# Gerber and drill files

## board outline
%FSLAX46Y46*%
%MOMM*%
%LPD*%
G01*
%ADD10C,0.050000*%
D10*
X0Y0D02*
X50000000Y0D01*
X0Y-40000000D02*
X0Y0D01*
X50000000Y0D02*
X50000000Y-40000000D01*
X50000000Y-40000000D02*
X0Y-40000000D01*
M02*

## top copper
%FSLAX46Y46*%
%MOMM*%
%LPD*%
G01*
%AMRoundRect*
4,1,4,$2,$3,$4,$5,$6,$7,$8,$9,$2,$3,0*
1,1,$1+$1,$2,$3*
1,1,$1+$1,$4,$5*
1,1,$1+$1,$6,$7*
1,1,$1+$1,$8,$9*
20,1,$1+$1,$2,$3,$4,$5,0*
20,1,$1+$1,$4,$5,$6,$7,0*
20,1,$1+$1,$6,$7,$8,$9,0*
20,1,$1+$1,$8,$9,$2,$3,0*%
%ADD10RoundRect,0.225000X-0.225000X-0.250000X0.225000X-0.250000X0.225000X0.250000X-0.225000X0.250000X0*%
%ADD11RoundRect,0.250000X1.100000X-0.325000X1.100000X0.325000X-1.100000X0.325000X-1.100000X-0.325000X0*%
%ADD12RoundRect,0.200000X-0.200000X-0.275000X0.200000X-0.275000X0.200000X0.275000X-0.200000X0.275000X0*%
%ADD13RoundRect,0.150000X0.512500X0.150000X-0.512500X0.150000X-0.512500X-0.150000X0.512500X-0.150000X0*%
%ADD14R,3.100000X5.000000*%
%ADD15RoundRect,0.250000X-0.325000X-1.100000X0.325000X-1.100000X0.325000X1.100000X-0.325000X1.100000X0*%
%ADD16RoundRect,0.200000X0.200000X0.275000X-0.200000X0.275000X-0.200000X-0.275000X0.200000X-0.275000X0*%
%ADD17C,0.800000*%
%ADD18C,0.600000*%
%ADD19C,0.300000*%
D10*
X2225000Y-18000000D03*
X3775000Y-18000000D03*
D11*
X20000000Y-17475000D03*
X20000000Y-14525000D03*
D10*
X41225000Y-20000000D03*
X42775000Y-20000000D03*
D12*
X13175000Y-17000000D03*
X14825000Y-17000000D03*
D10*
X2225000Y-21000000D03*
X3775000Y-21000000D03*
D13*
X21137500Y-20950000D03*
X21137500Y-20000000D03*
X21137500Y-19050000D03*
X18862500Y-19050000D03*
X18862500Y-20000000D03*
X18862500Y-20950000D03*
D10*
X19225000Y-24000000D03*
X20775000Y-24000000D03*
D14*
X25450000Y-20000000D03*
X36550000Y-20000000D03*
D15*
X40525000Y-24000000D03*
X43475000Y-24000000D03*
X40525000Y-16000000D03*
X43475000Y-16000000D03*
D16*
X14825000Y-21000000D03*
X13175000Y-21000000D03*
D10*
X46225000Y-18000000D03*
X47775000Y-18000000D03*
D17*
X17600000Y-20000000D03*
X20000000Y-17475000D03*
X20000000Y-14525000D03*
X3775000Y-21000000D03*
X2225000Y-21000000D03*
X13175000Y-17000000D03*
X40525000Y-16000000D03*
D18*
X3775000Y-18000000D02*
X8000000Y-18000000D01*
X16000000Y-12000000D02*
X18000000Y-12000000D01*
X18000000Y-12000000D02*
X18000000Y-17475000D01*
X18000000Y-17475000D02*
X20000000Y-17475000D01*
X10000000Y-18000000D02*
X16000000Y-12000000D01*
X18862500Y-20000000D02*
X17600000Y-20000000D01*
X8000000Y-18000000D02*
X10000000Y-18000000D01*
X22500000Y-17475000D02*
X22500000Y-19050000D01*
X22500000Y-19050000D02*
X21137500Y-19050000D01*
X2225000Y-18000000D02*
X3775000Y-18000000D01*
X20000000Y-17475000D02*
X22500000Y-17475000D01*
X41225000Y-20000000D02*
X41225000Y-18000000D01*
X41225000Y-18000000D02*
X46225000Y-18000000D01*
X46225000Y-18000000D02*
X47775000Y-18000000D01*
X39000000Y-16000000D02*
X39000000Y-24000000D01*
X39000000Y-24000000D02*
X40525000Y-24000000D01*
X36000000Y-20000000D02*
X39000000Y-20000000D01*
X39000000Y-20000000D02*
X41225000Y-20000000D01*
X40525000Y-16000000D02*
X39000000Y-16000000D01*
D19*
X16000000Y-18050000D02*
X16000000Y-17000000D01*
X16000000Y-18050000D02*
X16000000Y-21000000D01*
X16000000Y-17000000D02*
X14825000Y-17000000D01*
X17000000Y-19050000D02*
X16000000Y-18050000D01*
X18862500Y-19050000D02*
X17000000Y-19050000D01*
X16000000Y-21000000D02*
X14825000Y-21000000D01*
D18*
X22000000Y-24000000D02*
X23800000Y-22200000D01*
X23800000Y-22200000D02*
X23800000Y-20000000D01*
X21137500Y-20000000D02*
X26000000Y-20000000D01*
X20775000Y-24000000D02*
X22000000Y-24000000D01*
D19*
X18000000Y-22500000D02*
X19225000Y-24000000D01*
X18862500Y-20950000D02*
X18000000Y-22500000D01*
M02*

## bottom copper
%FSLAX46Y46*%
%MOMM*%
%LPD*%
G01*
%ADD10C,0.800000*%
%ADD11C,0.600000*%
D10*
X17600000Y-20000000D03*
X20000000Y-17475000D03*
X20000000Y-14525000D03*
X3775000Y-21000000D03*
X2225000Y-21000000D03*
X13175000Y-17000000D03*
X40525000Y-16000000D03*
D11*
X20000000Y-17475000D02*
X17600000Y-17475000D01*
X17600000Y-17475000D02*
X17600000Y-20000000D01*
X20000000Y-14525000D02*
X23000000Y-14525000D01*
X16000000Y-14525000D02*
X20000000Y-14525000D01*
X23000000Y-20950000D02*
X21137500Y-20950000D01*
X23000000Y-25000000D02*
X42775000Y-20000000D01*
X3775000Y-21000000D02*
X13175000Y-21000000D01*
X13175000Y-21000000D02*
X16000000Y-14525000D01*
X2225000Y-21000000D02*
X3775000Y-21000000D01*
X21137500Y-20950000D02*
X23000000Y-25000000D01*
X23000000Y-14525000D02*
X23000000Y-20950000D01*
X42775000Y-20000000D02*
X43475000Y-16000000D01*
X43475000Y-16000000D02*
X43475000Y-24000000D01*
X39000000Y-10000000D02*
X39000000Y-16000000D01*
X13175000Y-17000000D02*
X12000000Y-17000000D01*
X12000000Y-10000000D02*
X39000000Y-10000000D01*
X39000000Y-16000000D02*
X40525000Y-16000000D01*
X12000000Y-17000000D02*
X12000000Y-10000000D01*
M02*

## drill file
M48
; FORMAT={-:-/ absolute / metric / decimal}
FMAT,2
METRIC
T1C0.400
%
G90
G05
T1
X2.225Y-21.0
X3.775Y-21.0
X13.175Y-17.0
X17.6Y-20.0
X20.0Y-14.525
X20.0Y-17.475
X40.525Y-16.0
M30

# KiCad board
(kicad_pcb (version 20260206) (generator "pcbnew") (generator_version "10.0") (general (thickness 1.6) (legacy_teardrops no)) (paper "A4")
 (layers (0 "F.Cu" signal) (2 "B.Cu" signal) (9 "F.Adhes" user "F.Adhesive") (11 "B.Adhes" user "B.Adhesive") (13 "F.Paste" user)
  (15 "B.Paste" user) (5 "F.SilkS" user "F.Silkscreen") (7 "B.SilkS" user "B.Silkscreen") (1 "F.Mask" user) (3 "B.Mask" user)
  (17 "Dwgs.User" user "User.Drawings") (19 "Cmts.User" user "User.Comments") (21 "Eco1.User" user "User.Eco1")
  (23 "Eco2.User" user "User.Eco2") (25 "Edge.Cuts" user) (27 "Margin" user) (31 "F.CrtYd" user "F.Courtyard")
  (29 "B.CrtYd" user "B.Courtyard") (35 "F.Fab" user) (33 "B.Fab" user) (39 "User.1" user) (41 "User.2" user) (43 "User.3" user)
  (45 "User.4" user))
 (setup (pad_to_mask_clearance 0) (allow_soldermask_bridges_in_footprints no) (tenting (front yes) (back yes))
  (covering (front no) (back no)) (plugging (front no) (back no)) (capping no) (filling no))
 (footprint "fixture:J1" (layer "F.Cu") (at 3 18)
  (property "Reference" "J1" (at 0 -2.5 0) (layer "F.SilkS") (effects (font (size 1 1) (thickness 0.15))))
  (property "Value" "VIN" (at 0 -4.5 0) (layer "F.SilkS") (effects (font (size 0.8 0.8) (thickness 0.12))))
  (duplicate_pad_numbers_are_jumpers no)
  (pad "1" smd roundrect (at -0.775 0) (size 0.9 0.95) (layers "F.Cu" "F.Mask" "F.Paste") (roundrect_rratio 0.25) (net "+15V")
   (thermal_bridge_angle 45))
  (pad "2" smd roundrect (at 0.775 0) (size 0.9 0.95) (layers "F.Cu" "F.Mask" "F.Paste") (roundrect_rratio 0.25) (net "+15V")
   (thermal_bridge_angle 45)))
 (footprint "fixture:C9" (layer "F.Cu") (at 20 16 90)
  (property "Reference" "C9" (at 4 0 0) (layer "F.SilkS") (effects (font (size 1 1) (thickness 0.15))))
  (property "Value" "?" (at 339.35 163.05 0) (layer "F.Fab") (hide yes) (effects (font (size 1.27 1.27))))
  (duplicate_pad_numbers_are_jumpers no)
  (pad "1" smd roundrect (at -1.475 0 90) (size 1.15 2.7) (layers "F.Cu" "F.Mask" "F.Paste") (roundrect_rratio 0.217391) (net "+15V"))
  (pad "2" smd roundrect (at 1.475 0 90) (size 1.15 2.7) (layers "F.Cu" "F.Mask" "F.Paste") (roundrect_rratio 0.217391) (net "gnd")))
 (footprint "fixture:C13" (layer "F.Cu") (at 42 20)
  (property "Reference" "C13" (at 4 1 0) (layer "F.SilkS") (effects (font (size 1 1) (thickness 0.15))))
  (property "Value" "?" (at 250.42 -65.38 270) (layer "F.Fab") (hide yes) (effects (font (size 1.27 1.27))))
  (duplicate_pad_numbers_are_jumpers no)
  (pad "1" smd roundrect (at -0.775 0) (size 0.9 0.95) (layers "F.Cu" "F.Mask" "F.Paste") (roundrect_rratio 0.25) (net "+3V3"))
  (pad "2" smd roundrect (at 0.775 0) (size 0.9 0.95) (layers "F.Cu" "F.Mask" "F.Paste") (roundrect_rratio 0.25) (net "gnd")))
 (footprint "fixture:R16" (layer "F.Cu") (at 14 17)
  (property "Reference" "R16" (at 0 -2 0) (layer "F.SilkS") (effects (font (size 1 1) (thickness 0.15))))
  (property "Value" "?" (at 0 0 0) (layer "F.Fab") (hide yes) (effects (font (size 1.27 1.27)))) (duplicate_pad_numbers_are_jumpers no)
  (pad "1" smd roundrect (at -0.825 0) (size 0.8 0.95) (layers "F.Cu" "F.Mask" "F.Paste") (roundrect_rratio 0.25) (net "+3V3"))
  (pad "2" smd roundrect (at 0.825 0) (size 0.8 0.95) (layers "F.Cu" "F.Mask" "F.Paste") (roundrect_rratio 0.25) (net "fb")))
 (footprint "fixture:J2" (layer "F.Cu") (at 3 21)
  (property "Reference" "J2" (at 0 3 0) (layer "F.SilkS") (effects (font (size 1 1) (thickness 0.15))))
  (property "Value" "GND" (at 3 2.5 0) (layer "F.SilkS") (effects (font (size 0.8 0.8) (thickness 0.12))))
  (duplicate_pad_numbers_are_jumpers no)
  (pad "1" smd roundrect (at -0.775 0) (size 0.9 0.95) (layers "F.Cu" "F.Mask" "F.Paste") (roundrect_rratio 0.25) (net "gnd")
   (thermal_bridge_angle 45))
  (pad "2" smd roundrect (at 0.775 0) (size 0.9 0.95) (layers "F.Cu" "F.Mask" "F.Paste") (roundrect_rratio 0.25) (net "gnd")
   (thermal_bridge_angle 45)))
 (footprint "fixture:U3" (layer "F.Cu") (at 20 20 180)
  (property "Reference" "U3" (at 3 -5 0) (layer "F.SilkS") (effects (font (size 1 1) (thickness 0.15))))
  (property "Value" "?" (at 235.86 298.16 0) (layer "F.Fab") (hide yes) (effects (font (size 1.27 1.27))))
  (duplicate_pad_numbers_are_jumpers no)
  (pad "1" smd roundrect (at -1.1375 -0.95 180) (size 1.325 0.6) (layers "F.Cu" "F.Mask" "F.Paste") (roundrect_rratio 0.25) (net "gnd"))
  (pad "2" smd roundrect (at -1.1375 0 180) (size 1.325 0.6) (layers "F.Cu" "F.Mask" "F.Paste") (roundrect_rratio 0.25) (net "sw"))
  (pad "3" smd roundrect (at -1.1375 0.95 180) (size 1.325 0.6) (layers "F.Cu" "F.Mask" "F.Paste") (roundrect_rratio 0.25) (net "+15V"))
  (pad "4" smd roundrect (at 1.1375 0.95 180) (size 1.325 0.6) (layers "F.Cu" "F.Mask" "F.Paste") (roundrect_rratio 0.25) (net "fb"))
  (pad "5" smd roundrect (at 1.1375 0 180) (size 1.325 0.6) (layers "F.Cu" "F.Mask" "F.Paste") (roundrect_rratio 0.25) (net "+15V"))
  (pad "6" smd roundrect (at 1.1375 -0.95 180) (size 1.325 0.6) (layers "F.Cu" "F.Mask" "F.Paste") (roundrect_rratio 0.25) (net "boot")))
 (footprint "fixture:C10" (layer "F.Cu") (at 20 24)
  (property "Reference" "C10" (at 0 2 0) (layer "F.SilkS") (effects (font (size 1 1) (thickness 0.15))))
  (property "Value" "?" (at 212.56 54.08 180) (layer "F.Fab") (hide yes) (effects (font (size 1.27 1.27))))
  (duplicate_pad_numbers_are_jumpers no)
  (pad "1" smd roundrect (at -0.775 0) (size 0.9 0.95) (layers "F.Cu" "F.Mask" "F.Paste") (roundrect_rratio 0.25) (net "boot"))
  (pad "2" smd roundrect (at 0.775 0) (size 0.9 0.95) (layers "F.Cu" "F.Mask" "F.Paste") (roundrect_rratio 0.25) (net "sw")))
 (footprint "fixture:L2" (layer "F.Cu") (at 31 20)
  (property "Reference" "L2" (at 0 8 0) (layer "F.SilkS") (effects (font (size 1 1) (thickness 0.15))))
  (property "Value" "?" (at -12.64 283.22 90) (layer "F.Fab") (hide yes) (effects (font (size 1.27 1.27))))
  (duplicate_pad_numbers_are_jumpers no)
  (pad "1" smd rect (at -5.55 0) (size 3.1 5) (layers "F.Cu" "F.Mask" "F.Paste") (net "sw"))
  (pad "2" smd rect (at 5.55 0) (size 3.1 5) (layers "F.Cu" "F.Mask" "F.Paste") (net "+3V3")))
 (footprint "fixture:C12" (layer "F.Cu") (at 42 24)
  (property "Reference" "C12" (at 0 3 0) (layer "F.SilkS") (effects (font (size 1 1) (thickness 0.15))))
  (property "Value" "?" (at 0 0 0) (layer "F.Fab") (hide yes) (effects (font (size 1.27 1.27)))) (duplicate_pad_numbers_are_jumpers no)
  (pad "1" smd roundrect (at -1.475 0) (size 1.15 2.7) (layers "F.Cu" "F.Mask" "F.Paste") (roundrect_rratio 0.217391) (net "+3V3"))
  (pad "2" smd roundrect (at 1.475 0) (size 1.15 2.7) (layers "F.Cu" "F.Mask" "F.Paste") (roundrect_rratio 0.217391) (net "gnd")))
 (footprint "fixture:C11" (layer "F.Cu") (at 42 16)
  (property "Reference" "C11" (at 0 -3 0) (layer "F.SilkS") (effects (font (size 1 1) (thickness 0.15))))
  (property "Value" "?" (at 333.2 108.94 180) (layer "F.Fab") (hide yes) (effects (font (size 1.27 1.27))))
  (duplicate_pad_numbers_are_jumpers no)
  (pad "1" smd roundrect (at -1.475 0) (size 1.15 2.7) (layers "F.Cu" "F.Mask" "F.Paste") (roundrect_rratio 0.217391) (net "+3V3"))
  (pad "2" smd roundrect (at 1.475 0) (size 1.15 2.7) (layers "F.Cu" "F.Mask" "F.Paste") (roundrect_rratio 0.217391) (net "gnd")))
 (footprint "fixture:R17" (layer "F.Cu") (at 14 21 180)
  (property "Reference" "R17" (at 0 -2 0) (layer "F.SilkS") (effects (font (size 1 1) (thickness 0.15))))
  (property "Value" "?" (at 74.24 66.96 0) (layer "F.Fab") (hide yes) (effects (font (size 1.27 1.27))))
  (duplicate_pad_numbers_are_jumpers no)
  (pad "1" smd roundrect (at -0.825 0 180) (size 0.8 0.95) (layers "F.Cu" "F.Mask" "F.Paste") (roundrect_rratio 0.25) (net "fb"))
  (pad "2" smd roundrect (at 0.825 0 180) (size 0.8 0.95) (layers "F.Cu" "F.Mask" "F.Paste") (roundrect_rratio 0.25) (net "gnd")))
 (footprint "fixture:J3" (layer "F.Cu") (at 47 18)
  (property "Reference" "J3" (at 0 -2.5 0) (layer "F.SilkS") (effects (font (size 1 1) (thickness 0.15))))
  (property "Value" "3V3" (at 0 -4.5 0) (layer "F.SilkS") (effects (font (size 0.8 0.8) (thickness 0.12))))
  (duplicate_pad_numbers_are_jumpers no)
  (pad "1" smd roundrect (at -0.775 0) (size 0.9 0.95) (layers "F.Cu" "F.Mask" "F.Paste") (roundrect_rratio 0.25) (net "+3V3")
   (thermal_bridge_angle 45))
  (pad "2" smd roundrect (at 0.775 0) (size 0.9 0.95) (layers "F.Cu" "F.Mask" "F.Paste") (roundrect_rratio 0.25) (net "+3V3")
   (thermal_bridge_angle 45)))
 (gr_line (start 0 0) (end 50 0) (stroke (width 0.05) (type default)) (layer "Edge.Cuts"))
 (gr_line (start 0 40) (end 0 0) (stroke (width 0.05) (type default)) (layer "Edge.Cuts"))
 (gr_line (start 50 0) (end 50 40) (stroke (width 0.05) (type default)) (layer "Edge.Cuts"))
 (gr_line (start 50 40) (end 0 40) (stroke (width 0.05) (type default)) (layer "Edge.Cuts"))
 (segment (start 3.775 18) (end 8 18) (width 0.6) (layer "F.Cu") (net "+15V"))
 (segment (start 16 12) (end 18 12) (width 0.6) (layer "F.Cu") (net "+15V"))
 (segment (start 18 12) (end 18 17.475) (width 0.6) (layer "F.Cu") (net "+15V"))
 (segment (start 18 17.475) (end 20 17.475) (width 0.6) (layer "F.Cu") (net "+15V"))
 (segment (start 10 18) (end 16 12) (width 0.6) (layer "F.Cu") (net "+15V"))
 (segment (start 18.8625 20) (end 17.6 20) (width 0.6) (layer "F.Cu") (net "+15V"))
 (segment (start 8 18) (end 10 18) (width 0.6) (layer "F.Cu") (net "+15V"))
 (segment (start 22.5 17.475) (end 22.5 19.05) (width 0.6) (layer "F.Cu") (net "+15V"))
 (segment (start 22.5 19.05) (end 21.1375 19.05) (width 0.6) (layer "F.Cu") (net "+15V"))
 (segment (start 2.225 18) (end 3.775 18) (width 0.6) (layer "F.Cu") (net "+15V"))
 (segment (start 20 17.475) (end 22.5 17.475) (width 0.6) (layer "F.Cu") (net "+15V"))
 (via (at 17.6 20) (size 0.8) (drill 0.4) (layers "F.Cu" "B.Cu") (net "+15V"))
 (via (at 20 17.475) (size 0.8) (drill 0.4) (layers "F.Cu" "B.Cu") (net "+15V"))
 (segment (start 20 17.475) (end 17.6 17.475) (width 0.6) (layer "B.Cu") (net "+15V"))
 (segment (start 17.6 17.475) (end 17.6 20) (width 0.6) (layer "B.Cu") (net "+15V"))
 (via (at 20 14.525) (size 0.8) (drill 0.4) (layers "F.Cu" "B.Cu") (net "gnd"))
 (via (at 3.775 21) (size 0.8) (drill 0.4) (layers "F.Cu" "B.Cu") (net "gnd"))
 (via (at 2.225 21) (size 0.8) (drill 0.4) (layers "F.Cu" "B.Cu") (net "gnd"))
 (segment (start 20 14.525) (end 23 14.525) (width 0.6) (layer "B.Cu") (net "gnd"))
 (segment (start 16 14.525) (end 20 14.525) (width 0.6) (layer "B.Cu") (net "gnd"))
 (segment (start 23 20.95) (end 21.1375 20.95) (width 0.6) (layer "B.Cu") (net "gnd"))
 (segment (start 23 25) (end 42.775 20) (width 0.6) (layer "B.Cu") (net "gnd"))
 (segment (start 3.775 21) (end 13.175 21) (width 0.6) (layer "B.Cu") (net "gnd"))
 (segment (start 13.175 21) (end 16 14.525) (width 0.6) (layer "B.Cu") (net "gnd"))
 (segment (start 2.225 21) (end 3.775 21) (width 0.6) (layer "B.Cu") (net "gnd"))
 (segment (start 21.1375 20.95) (end 23 25) (width 0.6) (layer "B.Cu") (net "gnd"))
 (segment (start 23 14.525) (end 23 20.95) (width 0.6) (layer "B.Cu") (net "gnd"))
 (segment (start 42.775 20) (end 43.475 16) (width 0.6) (layer "B.Cu") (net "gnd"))
 (segment (start 43.475 16) (end 43.475 24) (width 0.6) (layer "B.Cu") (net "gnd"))
 (segment (start 41.225 20) (end 41.225 18) (width 0.6) (layer "F.Cu") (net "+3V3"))
 (segment (start 41.225 18) (end 46.225 18) (width 0.6) (layer "F.Cu") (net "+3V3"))
 (segment (start 46.225 18) (end 47.775 18) (width 0.6) (layer "F.Cu") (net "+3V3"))
 (segment (start 39 16) (end 39 24) (width 0.6) (layer "F.Cu") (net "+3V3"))
 (segment (start 39 24) (end 40.525 24) (width 0.6) (layer "F.Cu") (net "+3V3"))
 (segment (start 36 20) (end 39 20) (width 0.6) (layer "F.Cu") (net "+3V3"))
 (segment (start 39 20) (end 41.225 20) (width 0.6) (layer "F.Cu") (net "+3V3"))
 (segment (start 40.525 16) (end 39 16) (width 0.6) (layer "F.Cu") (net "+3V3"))
 (via (at 13.175 17) (size 0.8) (drill 0.4) (layers "F.Cu" "B.Cu") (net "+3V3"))
 (via (at 40.525 16) (size 0.8) (drill 0.4) (layers "F.Cu" "B.Cu") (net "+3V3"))
 (segment (start 39 10) (end 39 16) (width 0.6) (layer "B.Cu") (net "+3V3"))
 (segment (start 13.175 17) (end 12 17) (width 0.6) (layer "B.Cu") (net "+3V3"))
 (segment (start 12 10) (end 39 10) (width 0.6) (layer "B.Cu") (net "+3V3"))
 (segment (start 39 16) (end 40.525 16) (width 0.6) (layer "B.Cu") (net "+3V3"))
 (segment (start 12 17) (end 12 10) (width 0.6) (layer "B.Cu") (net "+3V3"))
 (segment (start 16 18.05) (end 16 17) (width 0.3) (layer "F.Cu") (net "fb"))
 (segment (start 16 18.05) (end 16 21) (width 0.3) (layer "F.Cu") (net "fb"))
 (segment (start 16 17) (end 14.825 17) (width 0.3) (layer "F.Cu") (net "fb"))
 (segment (start 17 19.05) (end 16 18.05) (width 0.3) (layer "F.Cu") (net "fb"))
 (segment (start 18.8625 19.05) (end 17 19.05) (width 0.3) (layer "F.Cu") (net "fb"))
 (segment (start 16 21) (end 14.825 21) (width 0.3) (layer "F.Cu") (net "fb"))
 (segment (start 22 24) (end 23.8 22.2) (width 0.6) (layer "F.Cu") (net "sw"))
 (segment (start 23.8 22.2) (end 23.8 20) (width 0.6) (layer "F.Cu") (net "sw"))
 (segment (start 21.1375 20) (end 26 20) (width 0.6) (layer "F.Cu") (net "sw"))
 (segment (start 20.775 24) (end 22 24) (width 0.6) (layer "F.Cu") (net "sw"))
 (segment (start 18 22.5) (end 19.225 24) (width 0.3) (layer "F.Cu") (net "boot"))
 (segment (start 18.8625 20.95) (end 18 22.5) (width 0.3) (layer "F.Cu") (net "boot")))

